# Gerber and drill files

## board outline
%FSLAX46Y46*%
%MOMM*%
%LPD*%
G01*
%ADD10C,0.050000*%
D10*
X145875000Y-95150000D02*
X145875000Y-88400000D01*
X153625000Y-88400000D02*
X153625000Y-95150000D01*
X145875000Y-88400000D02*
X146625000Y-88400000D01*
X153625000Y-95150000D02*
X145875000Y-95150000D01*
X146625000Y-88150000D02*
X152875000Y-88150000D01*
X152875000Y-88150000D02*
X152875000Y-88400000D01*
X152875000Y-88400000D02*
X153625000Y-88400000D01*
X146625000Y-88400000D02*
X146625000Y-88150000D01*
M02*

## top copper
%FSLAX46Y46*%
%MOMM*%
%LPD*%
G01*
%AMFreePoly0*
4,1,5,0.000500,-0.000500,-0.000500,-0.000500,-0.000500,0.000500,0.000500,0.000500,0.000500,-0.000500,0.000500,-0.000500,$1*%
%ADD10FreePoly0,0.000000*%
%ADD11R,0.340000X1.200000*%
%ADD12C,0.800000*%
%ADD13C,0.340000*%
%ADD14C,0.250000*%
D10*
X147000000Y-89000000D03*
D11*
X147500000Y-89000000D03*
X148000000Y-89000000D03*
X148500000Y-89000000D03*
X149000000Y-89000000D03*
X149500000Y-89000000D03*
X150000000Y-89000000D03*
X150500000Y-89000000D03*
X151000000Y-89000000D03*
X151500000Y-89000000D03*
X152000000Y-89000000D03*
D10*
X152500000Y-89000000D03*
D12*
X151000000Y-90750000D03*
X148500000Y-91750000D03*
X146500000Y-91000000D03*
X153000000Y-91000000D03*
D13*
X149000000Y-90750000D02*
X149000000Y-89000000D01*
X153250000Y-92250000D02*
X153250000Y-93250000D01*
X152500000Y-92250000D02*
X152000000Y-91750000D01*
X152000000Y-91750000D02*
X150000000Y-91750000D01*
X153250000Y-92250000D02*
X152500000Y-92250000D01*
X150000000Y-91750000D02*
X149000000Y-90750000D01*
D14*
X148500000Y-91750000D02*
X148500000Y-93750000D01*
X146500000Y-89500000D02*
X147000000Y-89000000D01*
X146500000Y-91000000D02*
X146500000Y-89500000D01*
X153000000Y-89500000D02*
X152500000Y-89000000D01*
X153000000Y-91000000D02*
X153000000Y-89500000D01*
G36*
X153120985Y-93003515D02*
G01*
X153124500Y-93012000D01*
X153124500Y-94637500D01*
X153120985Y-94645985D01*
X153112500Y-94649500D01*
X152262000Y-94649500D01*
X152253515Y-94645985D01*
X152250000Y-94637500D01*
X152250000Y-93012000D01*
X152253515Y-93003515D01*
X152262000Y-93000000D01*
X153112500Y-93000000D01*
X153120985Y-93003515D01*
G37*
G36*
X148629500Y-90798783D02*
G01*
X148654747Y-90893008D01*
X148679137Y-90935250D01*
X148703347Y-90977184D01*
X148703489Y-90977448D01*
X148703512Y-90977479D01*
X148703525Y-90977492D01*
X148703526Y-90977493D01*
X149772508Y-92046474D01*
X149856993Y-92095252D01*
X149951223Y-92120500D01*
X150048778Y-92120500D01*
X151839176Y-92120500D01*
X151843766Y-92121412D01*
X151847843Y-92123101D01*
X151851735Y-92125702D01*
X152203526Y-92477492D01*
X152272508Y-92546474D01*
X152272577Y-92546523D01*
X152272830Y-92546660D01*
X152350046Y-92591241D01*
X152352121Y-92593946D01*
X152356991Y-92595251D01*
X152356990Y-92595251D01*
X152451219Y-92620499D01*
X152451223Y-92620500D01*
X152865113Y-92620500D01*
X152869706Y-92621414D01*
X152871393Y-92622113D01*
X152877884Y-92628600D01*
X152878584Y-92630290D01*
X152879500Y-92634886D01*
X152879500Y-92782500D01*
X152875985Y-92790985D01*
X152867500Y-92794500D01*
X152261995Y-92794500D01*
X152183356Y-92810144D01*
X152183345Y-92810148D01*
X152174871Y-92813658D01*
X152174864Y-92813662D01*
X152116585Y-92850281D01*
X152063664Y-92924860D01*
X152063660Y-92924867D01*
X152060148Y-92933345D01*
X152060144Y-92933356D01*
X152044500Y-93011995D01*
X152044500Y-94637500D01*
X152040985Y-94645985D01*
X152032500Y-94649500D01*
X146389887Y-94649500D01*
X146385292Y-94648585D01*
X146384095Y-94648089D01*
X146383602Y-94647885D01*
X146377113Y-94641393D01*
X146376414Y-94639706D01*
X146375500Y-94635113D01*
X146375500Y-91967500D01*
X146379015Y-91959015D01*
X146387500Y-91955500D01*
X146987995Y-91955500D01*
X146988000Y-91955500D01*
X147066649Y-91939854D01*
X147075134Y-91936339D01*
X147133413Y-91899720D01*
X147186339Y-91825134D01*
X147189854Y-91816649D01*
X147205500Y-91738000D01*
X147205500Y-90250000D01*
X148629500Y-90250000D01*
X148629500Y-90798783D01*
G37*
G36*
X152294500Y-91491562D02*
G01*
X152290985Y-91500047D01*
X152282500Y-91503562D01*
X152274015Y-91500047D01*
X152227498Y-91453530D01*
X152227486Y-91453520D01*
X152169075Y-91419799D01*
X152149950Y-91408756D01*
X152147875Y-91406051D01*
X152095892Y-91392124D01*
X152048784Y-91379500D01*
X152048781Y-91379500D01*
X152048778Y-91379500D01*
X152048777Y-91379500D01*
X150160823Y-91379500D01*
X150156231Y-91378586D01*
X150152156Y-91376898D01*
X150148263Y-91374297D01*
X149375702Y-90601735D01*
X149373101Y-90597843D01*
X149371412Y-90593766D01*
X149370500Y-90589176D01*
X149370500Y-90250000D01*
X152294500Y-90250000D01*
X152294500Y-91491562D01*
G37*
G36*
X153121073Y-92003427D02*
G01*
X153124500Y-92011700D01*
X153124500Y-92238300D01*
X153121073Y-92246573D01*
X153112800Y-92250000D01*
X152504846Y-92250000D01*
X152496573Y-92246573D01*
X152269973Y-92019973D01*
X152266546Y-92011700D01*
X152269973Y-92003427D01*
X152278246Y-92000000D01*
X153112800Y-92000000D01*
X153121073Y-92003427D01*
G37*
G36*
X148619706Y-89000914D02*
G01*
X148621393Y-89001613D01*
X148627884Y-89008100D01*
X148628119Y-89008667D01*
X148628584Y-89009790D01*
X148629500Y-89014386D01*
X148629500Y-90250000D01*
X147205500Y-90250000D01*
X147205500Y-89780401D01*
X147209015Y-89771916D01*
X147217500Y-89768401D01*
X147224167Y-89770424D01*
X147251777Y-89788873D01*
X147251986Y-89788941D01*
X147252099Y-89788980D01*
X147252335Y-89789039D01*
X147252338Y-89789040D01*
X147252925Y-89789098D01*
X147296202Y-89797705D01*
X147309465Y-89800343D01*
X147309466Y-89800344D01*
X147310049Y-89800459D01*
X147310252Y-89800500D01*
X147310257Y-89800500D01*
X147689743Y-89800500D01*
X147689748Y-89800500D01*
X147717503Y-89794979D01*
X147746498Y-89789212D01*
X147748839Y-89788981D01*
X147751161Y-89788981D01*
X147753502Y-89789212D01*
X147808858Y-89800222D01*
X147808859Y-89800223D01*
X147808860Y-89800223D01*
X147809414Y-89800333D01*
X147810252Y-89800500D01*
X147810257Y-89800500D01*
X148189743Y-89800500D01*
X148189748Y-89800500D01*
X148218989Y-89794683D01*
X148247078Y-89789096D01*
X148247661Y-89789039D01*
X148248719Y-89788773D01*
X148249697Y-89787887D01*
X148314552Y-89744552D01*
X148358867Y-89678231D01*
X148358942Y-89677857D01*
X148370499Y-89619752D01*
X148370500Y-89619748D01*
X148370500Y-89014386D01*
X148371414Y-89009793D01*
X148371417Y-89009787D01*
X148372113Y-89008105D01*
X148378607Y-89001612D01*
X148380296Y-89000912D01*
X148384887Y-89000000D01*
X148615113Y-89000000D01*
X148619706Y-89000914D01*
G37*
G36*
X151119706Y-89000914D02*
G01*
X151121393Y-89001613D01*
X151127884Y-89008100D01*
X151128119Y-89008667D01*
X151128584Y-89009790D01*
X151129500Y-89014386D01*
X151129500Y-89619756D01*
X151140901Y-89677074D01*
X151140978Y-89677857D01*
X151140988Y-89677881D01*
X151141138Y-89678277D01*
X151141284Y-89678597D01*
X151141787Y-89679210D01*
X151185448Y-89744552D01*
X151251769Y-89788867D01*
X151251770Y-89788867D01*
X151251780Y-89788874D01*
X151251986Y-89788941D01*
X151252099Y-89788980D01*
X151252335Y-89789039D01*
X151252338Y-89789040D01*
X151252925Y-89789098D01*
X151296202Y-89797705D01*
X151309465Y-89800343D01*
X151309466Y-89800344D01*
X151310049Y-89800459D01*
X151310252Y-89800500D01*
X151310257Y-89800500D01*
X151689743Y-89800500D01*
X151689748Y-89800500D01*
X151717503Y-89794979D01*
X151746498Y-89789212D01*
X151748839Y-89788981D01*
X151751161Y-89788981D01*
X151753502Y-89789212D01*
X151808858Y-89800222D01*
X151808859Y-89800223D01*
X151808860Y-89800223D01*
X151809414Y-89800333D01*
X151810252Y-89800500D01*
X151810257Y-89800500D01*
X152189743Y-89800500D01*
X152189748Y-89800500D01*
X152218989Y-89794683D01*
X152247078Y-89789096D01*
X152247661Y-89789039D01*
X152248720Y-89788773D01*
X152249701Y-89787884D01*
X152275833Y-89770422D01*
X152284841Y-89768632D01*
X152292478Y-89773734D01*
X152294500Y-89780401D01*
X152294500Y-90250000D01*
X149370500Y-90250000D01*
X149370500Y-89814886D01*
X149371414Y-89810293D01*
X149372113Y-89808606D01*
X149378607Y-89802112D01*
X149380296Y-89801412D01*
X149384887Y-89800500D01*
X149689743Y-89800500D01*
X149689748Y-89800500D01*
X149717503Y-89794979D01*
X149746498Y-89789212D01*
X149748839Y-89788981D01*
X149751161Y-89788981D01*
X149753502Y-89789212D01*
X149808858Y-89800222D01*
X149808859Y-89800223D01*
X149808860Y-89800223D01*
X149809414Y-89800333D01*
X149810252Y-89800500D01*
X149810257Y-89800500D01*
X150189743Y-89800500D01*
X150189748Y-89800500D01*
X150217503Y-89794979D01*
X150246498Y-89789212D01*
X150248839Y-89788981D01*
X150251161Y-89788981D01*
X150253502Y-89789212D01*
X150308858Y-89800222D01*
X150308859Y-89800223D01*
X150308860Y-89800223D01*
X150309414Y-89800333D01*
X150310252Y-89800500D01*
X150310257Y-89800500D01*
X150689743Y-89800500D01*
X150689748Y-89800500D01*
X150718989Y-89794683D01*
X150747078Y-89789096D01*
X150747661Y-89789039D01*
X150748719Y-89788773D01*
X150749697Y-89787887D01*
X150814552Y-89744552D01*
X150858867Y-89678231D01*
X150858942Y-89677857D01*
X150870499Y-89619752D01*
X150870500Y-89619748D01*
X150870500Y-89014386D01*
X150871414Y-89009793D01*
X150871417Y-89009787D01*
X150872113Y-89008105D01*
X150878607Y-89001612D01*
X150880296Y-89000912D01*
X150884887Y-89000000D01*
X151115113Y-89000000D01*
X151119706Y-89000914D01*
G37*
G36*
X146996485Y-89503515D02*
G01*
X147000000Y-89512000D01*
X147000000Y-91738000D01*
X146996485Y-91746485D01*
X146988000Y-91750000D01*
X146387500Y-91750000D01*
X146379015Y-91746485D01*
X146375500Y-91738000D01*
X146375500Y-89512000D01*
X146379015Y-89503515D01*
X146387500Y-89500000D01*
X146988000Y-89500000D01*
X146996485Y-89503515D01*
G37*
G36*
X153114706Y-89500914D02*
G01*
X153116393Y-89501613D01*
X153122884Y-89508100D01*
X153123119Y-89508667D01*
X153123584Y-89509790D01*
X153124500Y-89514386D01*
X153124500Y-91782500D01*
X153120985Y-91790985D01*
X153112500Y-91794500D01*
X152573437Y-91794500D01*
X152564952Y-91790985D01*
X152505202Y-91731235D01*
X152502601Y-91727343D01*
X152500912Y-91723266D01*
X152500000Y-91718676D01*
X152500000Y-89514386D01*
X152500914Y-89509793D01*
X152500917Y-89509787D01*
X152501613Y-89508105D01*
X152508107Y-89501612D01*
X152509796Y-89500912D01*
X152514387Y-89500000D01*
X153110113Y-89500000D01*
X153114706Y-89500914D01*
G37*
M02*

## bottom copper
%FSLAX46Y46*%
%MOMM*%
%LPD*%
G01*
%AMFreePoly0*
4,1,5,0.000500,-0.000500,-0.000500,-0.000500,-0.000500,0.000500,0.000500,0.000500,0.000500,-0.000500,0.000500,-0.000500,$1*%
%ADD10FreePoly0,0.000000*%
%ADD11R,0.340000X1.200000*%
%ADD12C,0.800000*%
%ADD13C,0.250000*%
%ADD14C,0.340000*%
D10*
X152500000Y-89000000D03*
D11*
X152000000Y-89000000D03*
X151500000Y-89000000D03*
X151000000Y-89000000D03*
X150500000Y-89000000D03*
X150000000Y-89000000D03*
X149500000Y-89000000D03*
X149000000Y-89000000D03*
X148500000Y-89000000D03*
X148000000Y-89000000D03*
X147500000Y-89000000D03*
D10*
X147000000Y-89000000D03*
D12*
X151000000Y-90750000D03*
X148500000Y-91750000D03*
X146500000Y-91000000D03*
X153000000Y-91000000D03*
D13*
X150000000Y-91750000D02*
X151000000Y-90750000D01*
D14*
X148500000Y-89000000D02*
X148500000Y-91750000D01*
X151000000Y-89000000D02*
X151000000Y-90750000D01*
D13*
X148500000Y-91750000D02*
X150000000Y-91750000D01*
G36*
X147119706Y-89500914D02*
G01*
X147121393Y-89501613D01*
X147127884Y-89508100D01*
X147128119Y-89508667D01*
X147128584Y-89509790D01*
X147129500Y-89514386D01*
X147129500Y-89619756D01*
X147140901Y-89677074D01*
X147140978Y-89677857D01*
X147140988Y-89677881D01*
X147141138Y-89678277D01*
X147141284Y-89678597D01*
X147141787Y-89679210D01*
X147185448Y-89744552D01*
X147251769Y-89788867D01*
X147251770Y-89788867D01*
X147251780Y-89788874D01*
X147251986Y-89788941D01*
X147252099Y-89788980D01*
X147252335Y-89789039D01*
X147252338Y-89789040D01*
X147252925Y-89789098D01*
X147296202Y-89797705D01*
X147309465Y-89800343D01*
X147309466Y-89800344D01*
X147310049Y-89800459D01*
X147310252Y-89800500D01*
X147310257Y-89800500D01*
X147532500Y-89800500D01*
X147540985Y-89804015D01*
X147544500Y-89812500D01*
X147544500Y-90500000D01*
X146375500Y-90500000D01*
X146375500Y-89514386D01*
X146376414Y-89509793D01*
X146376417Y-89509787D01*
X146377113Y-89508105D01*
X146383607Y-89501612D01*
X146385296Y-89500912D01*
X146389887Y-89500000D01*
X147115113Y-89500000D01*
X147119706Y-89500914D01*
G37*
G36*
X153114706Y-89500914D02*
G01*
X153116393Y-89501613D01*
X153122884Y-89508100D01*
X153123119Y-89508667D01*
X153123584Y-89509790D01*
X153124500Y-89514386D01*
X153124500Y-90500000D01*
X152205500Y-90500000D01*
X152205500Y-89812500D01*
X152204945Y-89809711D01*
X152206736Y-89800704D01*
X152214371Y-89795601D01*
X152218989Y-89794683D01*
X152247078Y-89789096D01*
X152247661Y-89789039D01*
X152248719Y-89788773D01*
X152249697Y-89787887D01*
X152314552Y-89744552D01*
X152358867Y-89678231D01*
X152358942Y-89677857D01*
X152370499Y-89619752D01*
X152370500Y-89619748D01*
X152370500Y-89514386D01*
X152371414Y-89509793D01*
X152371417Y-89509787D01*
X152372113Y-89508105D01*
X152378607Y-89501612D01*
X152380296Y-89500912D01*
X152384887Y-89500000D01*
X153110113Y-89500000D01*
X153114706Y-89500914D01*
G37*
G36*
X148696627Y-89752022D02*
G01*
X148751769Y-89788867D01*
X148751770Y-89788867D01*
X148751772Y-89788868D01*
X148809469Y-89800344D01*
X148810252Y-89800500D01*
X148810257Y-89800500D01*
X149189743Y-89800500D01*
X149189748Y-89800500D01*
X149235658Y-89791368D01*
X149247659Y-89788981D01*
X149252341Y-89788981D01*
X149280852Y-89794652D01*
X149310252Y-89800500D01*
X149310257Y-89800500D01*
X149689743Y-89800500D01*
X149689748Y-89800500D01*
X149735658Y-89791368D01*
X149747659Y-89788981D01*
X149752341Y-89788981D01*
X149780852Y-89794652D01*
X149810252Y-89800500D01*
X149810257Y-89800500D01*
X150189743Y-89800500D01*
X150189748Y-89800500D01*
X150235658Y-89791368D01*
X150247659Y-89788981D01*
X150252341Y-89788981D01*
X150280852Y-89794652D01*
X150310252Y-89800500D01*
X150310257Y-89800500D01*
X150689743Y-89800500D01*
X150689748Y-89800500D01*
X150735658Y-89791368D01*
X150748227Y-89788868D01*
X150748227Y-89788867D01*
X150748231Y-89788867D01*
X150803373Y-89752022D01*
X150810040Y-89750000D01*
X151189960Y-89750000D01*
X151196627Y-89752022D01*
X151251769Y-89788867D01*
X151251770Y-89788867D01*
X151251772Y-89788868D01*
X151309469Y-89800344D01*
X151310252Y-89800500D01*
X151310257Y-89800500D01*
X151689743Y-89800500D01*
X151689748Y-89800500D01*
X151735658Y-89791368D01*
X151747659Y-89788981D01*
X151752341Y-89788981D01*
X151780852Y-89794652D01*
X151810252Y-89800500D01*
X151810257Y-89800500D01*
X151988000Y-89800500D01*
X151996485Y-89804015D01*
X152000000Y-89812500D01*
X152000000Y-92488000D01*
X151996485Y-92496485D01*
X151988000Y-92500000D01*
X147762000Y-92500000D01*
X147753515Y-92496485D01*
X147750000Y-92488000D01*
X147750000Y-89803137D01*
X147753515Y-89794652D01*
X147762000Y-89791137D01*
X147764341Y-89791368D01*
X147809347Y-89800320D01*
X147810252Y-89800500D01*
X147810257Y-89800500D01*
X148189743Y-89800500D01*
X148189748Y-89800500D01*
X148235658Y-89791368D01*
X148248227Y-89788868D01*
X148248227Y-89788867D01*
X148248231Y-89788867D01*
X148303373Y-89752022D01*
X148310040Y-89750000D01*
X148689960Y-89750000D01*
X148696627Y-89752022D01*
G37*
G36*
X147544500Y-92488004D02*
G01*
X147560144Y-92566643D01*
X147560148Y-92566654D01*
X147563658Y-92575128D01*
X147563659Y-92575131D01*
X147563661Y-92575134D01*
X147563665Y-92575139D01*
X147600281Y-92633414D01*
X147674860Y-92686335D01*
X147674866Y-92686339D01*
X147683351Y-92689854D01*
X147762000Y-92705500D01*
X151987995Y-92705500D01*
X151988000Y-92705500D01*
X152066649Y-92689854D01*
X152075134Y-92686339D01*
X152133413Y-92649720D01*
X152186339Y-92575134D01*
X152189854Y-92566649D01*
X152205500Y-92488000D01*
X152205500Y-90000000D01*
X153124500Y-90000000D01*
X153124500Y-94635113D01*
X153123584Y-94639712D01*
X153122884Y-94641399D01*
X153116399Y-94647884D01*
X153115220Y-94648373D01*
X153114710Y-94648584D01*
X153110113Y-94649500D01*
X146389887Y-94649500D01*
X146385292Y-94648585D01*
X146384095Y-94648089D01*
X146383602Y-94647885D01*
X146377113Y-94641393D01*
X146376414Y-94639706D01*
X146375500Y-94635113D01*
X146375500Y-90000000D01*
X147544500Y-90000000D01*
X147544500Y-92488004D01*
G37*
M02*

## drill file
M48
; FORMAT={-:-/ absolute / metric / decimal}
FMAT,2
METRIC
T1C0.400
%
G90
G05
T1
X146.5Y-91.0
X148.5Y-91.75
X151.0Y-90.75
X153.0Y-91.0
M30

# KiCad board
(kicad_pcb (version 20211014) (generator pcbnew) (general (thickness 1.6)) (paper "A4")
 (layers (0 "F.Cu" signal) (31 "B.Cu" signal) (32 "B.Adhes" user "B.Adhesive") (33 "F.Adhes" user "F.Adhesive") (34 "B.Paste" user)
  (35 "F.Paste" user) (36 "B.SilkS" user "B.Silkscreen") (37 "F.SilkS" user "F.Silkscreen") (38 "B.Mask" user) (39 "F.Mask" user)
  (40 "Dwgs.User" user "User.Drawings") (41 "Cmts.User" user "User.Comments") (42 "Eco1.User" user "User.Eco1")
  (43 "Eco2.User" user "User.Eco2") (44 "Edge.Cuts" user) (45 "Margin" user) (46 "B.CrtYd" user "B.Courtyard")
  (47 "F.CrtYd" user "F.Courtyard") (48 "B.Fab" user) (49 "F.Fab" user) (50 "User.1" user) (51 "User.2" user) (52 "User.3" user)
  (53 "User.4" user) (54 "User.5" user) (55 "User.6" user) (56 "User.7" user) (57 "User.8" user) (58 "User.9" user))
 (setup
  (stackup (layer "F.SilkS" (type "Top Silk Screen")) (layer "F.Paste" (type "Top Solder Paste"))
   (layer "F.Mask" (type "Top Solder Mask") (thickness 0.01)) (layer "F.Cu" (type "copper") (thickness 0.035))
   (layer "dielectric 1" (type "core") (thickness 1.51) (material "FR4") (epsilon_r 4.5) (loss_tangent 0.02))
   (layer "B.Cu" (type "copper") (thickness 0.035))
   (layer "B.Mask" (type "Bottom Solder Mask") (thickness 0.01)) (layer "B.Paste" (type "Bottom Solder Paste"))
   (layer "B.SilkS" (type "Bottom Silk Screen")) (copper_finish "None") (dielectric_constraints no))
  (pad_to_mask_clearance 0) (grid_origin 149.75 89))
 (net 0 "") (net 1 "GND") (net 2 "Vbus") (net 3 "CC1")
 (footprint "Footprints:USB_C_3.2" (layer "F.Cu") (at 149.75 89)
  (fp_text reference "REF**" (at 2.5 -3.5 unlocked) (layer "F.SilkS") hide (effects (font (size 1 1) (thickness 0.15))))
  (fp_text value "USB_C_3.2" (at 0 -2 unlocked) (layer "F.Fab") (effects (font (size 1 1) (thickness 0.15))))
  (pad "A1" smd custom (at -2.75 0) (size 0.001 0.001) (layers "F.Cu" "F.Paste" "F.Mask") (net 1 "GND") (solder_mask_margin 0.1)
   (zone_connect 2) (options (clearance outline) (anchor rect)) (primitives))
  (pad "A2" smd rect (at -2.25 0) (size 0.34 1.2) (layers "F.Cu" "F.Paste" "F.Mask"))
  (pad "A3" smd rect (at -1.75 0) (size 0.34 1.2) (layers "F.Cu" "F.Paste" "F.Mask"))
  (pad "A4" smd rect (at -1.25 0) (size 0.34 1.2) (layers "F.Cu" "F.Paste" "F.Mask") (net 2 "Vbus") (zone_connect 2))
  (pad "A5" smd rect (at -0.75 0) (size 0.34 1.2) (layers "F.Cu" "F.Paste" "F.Mask") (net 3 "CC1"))
  (pad "A6" smd rect (at -0.25 0) (size 0.34 1.2) (layers "F.Cu" "F.Paste" "F.Mask"))
  (pad "A7" smd rect (at 0.25 0) (size 0.34 1.2) (layers "F.Cu" "F.Paste" "F.Mask"))
  (pad "A8" smd rect (at 0.75 0) (size 0.34 1.2) (layers "F.Cu" "F.Paste" "F.Mask"))
  (pad "A9" smd rect (at 1.25 0) (size 0.34 1.2) (layers "F.Cu" "F.Paste" "F.Mask") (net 2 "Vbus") (zone_connect 2))
  (pad "A10" smd rect (at 1.75 0) (size 0.34 1.2) (layers "F.Cu" "F.Paste" "F.Mask"))
  (pad "A11" smd rect (at 2.25 0) (size 0.34 1.2) (layers "F.Cu" "F.Paste" "F.Mask"))
  (pad "A12" smd custom (at 2.75 0) (size 0.001 0.001) (layers "F.Cu" "F.Paste" "F.Mask") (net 1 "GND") (solder_mask_margin 0.1)
   (zone_connect 2) (options (clearance outline) (anchor rect)) (primitives))
  (pad "B1" smd custom (at 2.75 0) (size 0.001 0.001) (layers "B.Cu" "B.Paste" "B.Mask") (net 1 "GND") (solder_mask_margin 0.1)
   (zone_connect 2) (options (clearance outline) (anchor rect)) (primitives))
  (pad "B2" smd rect (at 2.25 0) (size 0.34 1.2) (layers "B.Cu" "B.Paste" "B.Mask"))
  (pad "B3" smd rect (at 1.75 0) (size 0.34 1.2) (layers "B.Cu" "B.Paste" "B.Mask"))
  (pad "B4" smd rect (at 1.25 0) (size 0.34 1.2) (layers "B.Cu" "B.Paste" "B.Mask") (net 2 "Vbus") (zone_connect 2))
  (pad "B5" smd rect (at 0.75 0) (size 0.34 1.2) (layers "B.Cu" "B.Paste" "B.Mask"))
  (pad "B6" smd rect (at 0.25 0) (size 0.34 1.2) (layers "B.Cu" "B.Paste" "B.Mask"))
  (pad "B7" smd rect (at -0.25 0) (size 0.34 1.2) (layers "B.Cu" "B.Paste" "B.Mask"))
  (pad "B8" smd rect (at -0.75 0) (size 0.34 1.2) (layers "B.Cu" "B.Paste" "B.Mask"))
  (pad "B9" smd rect (at -1.25 0) (size 0.34 1.2) (layers "B.Cu" "B.Paste" "B.Mask") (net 2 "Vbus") (zone_connect 2))
  (pad "B10" smd rect (at -1.75 0) (size 0.34 1.2) (layers "B.Cu" "B.Paste" "B.Mask"))
  (pad "B11" smd rect (at -2.25 0) (size 0.34 1.2) (layers "B.Cu" "B.Paste" "B.Mask"))
  (pad "B12" smd custom (at -2.75 0) (size 0.001 0.001) (layers "B.Cu" "B.Paste" "B.Mask") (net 1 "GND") (solder_mask_margin 0.1)
   (zone_connect 2) (options (clearance outline) (anchor rect)) (primitives)))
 (gr_line (start 145.875 95.15) (end 145.875 88.4) (layer "Edge.Cuts") (width 0.05))
 (gr_line (start 153.625 88.4) (end 153.625 95.15) (layer "Edge.Cuts") (width 0.05))
 (gr_line (start 145.875 88.4) (end 146.625 88.4) (layer "Edge.Cuts") (width 0.05))
 (gr_line (start 153.625 95.15) (end 145.875 95.15) (layer "Edge.Cuts") (width 0.05))
 (gr_line (start 146.625 88.15) (end 152.875 88.15) (layer "Edge.Cuts") (width 0.05))
 (gr_line (start 152.875 88.15) (end 152.875 88.4) (layer "Edge.Cuts") (width 0.05))
 (gr_line (start 152.875 88.4) (end 153.625 88.4) (layer "Edge.Cuts") (width 0.05))
 (gr_line (start 146.625 88.4) (end 146.625 88.15) (layer "Edge.Cuts") (width 0.05))
 (segment (start 149 90.75) (end 149 89) (width 0.34) (layer "F.Cu") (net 3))
 (segment (start 153.25 92.25) (end 153.25 93.25) (width 0.34) (layer "F.Cu") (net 3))
 (segment (start 152.5 92.25) (end 152 91.75) (width 0.34) (layer "F.Cu") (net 3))
 (segment (start 152 91.75) (end 150 91.75) (width 0.34) (layer "F.Cu") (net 3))
 (segment (start 153.25 92.25) (end 152.5 92.25) (width 0.34) (layer "F.Cu") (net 3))
 (segment (start 150 91.75) (end 149 90.75) (width 0.34) (layer "F.Cu") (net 3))
 (segment (start 148.5 91.75) (end 148.5 93.75) (width 0.25) (layer "F.Cu") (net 2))
 (via (at 151 90.75) (size 0.8) (drill 0.4) (layers "F.Cu" "B.Cu") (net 2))
 (via (at 148.5 91.75) (size 0.8) (drill 0.4) (layers "F.Cu" "B.Cu") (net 2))
 (segment (start 150 91.75) (end 151 90.75) (width 0.25) (layer "B.Cu") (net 2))
 (segment (start 148.5 89) (end 148.5 91.75) (width 0.34) (layer "B.Cu") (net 2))
 (segment (start 151 89) (end 151 90.75) (width 0.34) (layer "B.Cu") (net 2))
 (segment (start 148.5 91.75) (end 150 91.75) (width 0.25) (layer "B.Cu") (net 2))
 (segment (start 146.5 89.5) (end 147 89) (width 0.25) (layer "F.Cu") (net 1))
 (segment (start 146.5 91) (end 146.5 89.5) (width 0.25) (layer "F.Cu") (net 1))
 (segment (start 153 89.5) (end 152.5 89) (width 0.25) (layer "F.Cu") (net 1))
 (segment (start 153 91) (end 153 89.5) (width 0.25) (layer "F.Cu") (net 1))
 (via (at 146.5 91) (size 0.8) (drill 0.4) (layers "F.Cu" "B.Cu") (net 1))
 (via (at 153 91) (size 0.8) (drill 0.4) (layers "F.Cu" "B.Cu") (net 1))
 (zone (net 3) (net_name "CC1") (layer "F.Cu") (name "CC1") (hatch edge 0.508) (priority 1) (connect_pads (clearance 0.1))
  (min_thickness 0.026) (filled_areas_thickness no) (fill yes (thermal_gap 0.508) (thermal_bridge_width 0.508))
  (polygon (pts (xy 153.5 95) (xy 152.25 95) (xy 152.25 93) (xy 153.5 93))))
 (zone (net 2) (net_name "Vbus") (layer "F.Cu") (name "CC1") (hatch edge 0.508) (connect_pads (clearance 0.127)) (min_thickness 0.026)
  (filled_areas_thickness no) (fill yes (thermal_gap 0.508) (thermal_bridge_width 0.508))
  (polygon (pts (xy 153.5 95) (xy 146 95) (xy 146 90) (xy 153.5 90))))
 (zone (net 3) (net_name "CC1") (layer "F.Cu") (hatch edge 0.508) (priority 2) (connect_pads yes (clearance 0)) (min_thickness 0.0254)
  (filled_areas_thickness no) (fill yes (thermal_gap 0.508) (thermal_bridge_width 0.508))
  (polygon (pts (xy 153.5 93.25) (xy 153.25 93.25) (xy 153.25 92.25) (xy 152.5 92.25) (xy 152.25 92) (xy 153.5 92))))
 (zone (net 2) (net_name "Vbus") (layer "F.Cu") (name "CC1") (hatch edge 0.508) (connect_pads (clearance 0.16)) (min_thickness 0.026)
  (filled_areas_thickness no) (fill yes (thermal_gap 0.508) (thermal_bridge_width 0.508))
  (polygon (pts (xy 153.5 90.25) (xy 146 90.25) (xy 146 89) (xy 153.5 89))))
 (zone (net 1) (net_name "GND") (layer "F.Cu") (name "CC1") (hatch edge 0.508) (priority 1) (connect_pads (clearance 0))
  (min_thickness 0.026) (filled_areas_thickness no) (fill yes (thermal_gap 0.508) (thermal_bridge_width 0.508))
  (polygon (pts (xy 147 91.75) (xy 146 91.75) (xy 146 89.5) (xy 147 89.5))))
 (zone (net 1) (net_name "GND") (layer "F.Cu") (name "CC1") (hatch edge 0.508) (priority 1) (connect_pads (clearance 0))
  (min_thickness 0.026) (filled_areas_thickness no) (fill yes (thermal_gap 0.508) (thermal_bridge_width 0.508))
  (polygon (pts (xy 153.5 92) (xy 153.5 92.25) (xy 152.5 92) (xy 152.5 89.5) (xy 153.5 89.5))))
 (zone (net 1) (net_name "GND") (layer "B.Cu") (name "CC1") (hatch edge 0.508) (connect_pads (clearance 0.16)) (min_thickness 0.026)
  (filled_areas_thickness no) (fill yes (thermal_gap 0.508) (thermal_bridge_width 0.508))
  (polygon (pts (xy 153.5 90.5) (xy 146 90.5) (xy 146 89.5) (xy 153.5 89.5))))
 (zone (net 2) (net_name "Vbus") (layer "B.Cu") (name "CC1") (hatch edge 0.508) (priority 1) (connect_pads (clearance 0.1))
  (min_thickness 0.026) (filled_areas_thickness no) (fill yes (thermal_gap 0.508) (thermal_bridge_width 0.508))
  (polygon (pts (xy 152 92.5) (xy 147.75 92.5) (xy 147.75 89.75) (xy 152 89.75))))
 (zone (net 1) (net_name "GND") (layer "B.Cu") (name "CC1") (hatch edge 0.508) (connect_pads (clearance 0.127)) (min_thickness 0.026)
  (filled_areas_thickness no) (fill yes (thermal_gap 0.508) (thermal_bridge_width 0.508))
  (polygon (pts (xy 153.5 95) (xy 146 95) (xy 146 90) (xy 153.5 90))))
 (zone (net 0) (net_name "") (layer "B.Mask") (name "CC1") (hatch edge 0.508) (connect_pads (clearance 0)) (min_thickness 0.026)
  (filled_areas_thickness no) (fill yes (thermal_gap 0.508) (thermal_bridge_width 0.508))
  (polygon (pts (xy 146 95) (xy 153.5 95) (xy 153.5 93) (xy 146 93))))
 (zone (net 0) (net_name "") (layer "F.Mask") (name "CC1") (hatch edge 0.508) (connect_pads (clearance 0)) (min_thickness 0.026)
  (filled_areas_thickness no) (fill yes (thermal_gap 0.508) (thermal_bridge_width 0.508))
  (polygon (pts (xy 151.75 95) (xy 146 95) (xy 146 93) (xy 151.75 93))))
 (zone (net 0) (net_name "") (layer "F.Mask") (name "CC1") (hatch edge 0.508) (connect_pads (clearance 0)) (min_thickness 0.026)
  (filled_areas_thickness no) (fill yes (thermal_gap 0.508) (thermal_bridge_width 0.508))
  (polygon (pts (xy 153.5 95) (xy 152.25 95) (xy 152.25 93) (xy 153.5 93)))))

